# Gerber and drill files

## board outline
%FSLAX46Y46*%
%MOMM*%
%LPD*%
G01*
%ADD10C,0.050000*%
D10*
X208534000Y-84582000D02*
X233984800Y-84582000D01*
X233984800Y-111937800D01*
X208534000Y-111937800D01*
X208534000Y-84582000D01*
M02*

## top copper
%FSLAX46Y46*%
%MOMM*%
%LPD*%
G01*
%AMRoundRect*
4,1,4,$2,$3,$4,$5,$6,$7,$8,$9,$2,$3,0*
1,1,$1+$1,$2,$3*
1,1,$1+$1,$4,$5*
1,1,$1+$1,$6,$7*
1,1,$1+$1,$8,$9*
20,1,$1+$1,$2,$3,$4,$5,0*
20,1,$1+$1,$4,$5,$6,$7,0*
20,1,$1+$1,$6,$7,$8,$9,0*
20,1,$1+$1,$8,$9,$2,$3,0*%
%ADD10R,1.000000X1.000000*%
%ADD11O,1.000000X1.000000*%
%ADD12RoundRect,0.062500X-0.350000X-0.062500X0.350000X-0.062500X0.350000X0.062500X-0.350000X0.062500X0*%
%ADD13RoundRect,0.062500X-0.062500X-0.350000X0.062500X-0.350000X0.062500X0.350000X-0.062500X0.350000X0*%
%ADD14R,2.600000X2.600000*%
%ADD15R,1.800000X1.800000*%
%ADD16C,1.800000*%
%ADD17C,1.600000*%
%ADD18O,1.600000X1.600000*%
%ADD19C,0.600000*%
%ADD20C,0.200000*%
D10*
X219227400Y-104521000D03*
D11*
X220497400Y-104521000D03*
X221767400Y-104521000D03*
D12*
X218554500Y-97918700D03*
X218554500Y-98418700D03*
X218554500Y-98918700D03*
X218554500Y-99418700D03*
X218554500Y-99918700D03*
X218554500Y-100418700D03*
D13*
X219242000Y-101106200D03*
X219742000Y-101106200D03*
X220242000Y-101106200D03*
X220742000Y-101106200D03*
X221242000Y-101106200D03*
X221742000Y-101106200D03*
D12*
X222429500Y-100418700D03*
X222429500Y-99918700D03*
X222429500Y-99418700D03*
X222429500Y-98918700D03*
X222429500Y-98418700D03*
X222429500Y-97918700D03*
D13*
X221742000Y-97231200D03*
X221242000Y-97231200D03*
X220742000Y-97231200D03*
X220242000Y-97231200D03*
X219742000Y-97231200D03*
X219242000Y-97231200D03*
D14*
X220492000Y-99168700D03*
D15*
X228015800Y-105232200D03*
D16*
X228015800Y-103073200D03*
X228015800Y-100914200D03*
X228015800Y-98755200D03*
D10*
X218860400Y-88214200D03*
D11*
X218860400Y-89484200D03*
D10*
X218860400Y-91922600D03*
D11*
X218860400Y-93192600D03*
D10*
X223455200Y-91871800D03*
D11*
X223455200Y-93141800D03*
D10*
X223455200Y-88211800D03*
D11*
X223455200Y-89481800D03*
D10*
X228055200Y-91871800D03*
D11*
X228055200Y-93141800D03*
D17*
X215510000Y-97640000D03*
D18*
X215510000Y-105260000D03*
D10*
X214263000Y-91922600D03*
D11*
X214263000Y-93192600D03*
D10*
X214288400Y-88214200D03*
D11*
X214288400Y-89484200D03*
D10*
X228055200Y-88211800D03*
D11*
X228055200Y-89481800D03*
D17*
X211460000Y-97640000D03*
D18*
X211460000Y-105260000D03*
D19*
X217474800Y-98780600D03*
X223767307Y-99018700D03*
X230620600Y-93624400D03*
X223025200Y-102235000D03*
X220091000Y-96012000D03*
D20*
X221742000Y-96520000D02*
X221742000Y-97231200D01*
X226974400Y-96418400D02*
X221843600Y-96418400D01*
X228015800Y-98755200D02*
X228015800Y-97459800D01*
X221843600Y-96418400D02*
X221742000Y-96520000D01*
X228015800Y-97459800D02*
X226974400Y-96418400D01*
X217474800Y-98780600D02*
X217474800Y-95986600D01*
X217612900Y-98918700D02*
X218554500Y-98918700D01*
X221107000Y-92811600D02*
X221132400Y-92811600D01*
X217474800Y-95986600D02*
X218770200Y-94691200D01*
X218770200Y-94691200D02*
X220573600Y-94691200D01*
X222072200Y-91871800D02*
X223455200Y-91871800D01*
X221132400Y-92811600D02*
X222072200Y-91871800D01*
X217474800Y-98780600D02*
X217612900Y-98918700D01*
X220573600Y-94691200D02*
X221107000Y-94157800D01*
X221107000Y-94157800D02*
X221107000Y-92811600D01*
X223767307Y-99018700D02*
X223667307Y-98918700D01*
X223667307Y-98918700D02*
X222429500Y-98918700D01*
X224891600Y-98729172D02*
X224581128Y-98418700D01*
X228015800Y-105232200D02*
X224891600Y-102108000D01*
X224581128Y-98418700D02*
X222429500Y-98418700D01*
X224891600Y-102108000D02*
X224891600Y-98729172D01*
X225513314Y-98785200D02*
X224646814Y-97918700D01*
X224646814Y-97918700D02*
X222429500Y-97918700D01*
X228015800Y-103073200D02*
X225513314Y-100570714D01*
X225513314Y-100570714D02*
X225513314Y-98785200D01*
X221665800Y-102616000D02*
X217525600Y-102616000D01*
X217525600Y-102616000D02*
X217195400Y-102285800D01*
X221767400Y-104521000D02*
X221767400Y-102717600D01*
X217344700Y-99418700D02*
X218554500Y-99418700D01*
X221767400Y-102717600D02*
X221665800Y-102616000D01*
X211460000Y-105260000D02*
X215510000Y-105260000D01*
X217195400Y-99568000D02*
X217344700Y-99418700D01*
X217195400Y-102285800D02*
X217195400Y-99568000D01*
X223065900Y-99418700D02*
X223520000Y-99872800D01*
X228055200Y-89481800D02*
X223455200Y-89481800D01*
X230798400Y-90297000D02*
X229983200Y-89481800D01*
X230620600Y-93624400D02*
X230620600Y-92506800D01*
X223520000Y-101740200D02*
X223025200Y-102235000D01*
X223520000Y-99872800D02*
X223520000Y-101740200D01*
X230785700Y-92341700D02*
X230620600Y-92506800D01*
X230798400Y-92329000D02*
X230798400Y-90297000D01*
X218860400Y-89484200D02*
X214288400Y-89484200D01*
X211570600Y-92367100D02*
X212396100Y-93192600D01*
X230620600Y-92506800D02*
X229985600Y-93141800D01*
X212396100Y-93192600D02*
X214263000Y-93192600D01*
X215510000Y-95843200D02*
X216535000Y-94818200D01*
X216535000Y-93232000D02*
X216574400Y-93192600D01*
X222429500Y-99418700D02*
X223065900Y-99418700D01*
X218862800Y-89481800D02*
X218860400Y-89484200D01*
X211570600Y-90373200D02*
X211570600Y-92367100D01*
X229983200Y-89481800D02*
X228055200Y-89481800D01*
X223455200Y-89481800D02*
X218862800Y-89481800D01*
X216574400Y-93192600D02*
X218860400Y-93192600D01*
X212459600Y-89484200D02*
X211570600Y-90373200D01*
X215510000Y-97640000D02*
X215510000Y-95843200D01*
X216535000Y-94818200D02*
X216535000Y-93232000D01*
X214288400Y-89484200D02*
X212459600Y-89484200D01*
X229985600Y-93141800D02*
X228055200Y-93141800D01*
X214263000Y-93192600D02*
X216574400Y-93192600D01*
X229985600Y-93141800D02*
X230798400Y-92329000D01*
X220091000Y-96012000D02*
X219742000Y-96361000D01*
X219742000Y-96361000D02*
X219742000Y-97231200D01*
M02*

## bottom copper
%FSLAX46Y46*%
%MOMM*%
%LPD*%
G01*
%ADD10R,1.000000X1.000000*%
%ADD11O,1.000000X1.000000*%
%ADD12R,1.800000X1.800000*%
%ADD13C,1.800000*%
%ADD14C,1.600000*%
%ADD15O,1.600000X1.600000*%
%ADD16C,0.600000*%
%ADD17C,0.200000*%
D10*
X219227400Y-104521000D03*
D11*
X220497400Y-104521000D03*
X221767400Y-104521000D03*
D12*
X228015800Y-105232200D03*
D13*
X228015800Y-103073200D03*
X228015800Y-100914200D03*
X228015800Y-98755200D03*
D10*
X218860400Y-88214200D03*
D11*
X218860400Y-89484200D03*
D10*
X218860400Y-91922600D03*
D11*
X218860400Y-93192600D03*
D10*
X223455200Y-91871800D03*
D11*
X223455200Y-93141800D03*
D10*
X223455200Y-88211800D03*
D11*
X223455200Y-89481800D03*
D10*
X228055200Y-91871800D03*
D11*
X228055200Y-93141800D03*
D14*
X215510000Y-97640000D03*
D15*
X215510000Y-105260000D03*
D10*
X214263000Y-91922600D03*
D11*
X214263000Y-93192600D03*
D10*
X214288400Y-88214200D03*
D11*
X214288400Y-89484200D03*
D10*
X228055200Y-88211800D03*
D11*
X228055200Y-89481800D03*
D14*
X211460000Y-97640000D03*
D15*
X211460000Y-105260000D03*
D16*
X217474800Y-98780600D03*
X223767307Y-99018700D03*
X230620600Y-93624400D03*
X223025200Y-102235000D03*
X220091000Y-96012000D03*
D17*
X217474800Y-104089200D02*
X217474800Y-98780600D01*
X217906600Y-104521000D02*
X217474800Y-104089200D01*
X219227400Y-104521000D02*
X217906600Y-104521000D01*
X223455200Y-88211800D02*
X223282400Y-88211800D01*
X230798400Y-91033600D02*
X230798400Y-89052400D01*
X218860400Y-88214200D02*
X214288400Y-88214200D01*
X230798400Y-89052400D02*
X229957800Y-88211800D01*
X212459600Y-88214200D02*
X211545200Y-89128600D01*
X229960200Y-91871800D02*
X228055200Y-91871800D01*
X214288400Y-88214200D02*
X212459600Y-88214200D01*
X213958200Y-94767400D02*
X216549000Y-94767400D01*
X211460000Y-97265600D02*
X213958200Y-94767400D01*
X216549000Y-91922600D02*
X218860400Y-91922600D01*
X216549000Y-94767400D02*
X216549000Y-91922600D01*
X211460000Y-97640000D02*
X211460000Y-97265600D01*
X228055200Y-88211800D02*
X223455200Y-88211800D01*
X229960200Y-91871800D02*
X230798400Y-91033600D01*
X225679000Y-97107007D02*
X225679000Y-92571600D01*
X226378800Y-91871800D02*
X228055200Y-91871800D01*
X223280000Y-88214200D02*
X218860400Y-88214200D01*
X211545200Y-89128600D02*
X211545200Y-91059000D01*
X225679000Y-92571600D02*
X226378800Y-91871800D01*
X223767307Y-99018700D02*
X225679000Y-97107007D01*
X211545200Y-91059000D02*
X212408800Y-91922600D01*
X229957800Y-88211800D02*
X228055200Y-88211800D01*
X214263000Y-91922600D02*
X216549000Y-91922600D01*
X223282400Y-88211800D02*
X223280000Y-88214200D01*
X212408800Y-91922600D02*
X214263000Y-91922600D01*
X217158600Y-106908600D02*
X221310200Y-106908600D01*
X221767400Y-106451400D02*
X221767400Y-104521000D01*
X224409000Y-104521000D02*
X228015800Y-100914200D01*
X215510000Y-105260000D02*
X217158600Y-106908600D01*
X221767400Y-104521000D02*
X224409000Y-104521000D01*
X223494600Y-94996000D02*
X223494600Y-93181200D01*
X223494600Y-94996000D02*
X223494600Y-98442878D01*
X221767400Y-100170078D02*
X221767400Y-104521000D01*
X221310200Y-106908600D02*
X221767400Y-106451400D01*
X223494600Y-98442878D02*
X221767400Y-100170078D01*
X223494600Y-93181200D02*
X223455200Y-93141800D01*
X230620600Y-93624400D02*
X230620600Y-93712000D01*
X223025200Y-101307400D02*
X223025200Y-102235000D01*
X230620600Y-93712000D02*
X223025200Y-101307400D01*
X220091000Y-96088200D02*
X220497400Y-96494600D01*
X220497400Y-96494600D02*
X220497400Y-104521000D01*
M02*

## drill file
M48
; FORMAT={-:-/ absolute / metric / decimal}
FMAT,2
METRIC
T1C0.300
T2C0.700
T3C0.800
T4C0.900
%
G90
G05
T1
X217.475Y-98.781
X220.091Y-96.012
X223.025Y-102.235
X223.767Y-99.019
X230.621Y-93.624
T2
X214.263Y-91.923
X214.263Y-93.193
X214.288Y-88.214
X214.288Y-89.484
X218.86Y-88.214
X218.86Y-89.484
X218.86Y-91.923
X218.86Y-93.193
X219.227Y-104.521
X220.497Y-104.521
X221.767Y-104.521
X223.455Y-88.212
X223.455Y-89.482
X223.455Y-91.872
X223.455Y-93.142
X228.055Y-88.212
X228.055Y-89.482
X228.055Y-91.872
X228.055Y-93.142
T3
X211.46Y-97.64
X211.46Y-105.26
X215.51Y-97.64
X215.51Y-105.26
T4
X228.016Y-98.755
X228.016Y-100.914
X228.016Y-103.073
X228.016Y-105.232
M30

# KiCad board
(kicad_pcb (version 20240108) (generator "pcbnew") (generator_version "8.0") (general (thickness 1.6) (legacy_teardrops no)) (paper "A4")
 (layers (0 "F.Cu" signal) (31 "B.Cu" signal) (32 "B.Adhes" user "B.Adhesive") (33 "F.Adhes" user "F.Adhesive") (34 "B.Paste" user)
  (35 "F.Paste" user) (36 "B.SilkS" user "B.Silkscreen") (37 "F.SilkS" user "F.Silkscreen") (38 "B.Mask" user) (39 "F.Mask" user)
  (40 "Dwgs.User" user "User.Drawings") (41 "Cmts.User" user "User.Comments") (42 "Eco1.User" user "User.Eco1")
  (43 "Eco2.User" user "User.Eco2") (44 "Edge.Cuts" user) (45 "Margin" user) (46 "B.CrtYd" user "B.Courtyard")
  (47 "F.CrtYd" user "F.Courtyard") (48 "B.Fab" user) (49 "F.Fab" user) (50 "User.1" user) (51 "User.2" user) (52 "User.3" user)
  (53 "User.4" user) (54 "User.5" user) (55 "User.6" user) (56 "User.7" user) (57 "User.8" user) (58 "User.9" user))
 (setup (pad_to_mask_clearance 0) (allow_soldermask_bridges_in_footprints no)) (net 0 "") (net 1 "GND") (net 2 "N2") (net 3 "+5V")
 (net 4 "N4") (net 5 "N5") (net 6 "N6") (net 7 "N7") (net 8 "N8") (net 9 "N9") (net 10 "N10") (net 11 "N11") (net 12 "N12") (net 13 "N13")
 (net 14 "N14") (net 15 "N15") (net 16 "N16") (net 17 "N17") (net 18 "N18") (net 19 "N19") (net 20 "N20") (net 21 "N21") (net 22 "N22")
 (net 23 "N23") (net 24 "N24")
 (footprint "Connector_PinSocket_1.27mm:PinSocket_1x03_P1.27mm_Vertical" (layer "F.Cu") (at 219.2274 104.521 90)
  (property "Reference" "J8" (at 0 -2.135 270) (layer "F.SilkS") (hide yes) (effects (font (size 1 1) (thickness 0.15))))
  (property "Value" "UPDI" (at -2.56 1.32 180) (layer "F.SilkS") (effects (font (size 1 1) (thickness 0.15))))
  (pad "1" thru_hole rect (at 0 0 90) (size 1 1) (drill 0.7) (layers "*.Cu" "*.Mask") (remove_unused_layers no) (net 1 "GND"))
  (pad "2" thru_hole oval (at 0 1.27 90) (size 1 1) (drill 0.7) (layers "*.Cu" "*.Mask") (remove_unused_layers no) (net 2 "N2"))
  (pad "3" thru_hole oval (at 0 2.54 90) (size 1 1) (drill 0.7) (layers "*.Cu" "*.Mask") (remove_unused_layers no) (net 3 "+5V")))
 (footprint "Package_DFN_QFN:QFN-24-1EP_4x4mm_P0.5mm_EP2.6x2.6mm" (layer "F.Cu") (at 220.492 99.1687)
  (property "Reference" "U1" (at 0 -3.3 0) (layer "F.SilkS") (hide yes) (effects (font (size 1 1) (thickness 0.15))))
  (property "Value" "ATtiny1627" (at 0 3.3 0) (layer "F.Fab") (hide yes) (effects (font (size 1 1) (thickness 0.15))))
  (pad "" smd roundrect (at -0.65 -0.65) (size 1.05 1.05) (layers "F.Paste") (roundrect_rratio 0.238095))
  (pad "" smd roundrect (at -0.65 0.65) (size 1.05 1.05) (layers "F.Paste") (roundrect_rratio 0.238095))
  (pad "" smd roundrect (at 0.65 -0.65) (size 1.05 1.05) (layers "F.Paste") (roundrect_rratio 0.238095))
  (pad "" smd roundrect (at 0.65 0.65) (size 1.05 1.05) (layers "F.Paste") (roundrect_rratio 0.238095))
  (pad "1" smd roundrect (at -1.9375 -1.25) (size 0.825 0.25) (layers "F.Cu" "F.Paste" "F.Mask") (roundrect_rratio 0.25) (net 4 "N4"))
  (pad "2" smd roundrect (at -1.9375 -0.75) (size 0.825 0.25) (layers "F.Cu" "F.Paste" "F.Mask") (roundrect_rratio 0.25) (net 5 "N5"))
  (pad "3" smd roundrect (at -1.9375 -0.25) (size 0.825 0.25) (layers "F.Cu" "F.Paste" "F.Mask") (roundrect_rratio 0.25) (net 1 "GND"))
  (pad "4" smd roundrect (at -1.9375 0.25) (size 0.825 0.25) (layers "F.Cu" "F.Paste" "F.Mask") (roundrect_rratio 0.25) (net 3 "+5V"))
  (pad "5" smd roundrect (at -1.9375 0.75) (size 0.825 0.25) (layers "F.Cu" "F.Paste" "F.Mask") (roundrect_rratio 0.25) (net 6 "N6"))
  (pad "6" smd roundrect (at -1.9375 1.25) (size 0.825 0.25) (layers "F.Cu" "F.Paste" "F.Mask") (roundrect_rratio 0.25) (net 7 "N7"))
  (pad "7" smd roundrect (at -1.25 1.9375) (size 0.25 0.825) (layers "F.Cu" "F.Paste" "F.Mask") (roundrect_rratio 0.25) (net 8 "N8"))
  (pad "8" smd roundrect (at -0.75 1.9375) (size 0.25 0.825) (layers "F.Cu" "F.Paste" "F.Mask") (roundrect_rratio 0.25) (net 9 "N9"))
  (pad "9" smd roundrect (at -0.25 1.9375) (size 0.25 0.825) (layers "F.Cu" "F.Paste" "F.Mask") (roundrect_rratio 0.25) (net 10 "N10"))
  (pad "10" smd roundrect (at 0.25 1.9375) (size 0.25 0.825) (layers "F.Cu" "F.Paste" "F.Mask") (roundrect_rratio 0.25) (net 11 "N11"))
  (pad "11" smd roundrect (at 0.75 1.9375) (size 0.25 0.825) (layers "F.Cu" "F.Paste" "F.Mask") (roundrect_rratio 0.25) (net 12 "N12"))
  (pad "12" smd roundrect (at 1.25 1.9375) (size 0.25 0.825) (layers "F.Cu" "F.Paste" "F.Mask") (roundrect_rratio 0.25) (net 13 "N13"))
  (pad "13" smd roundrect (at 1.9375 1.25) (size 0.825 0.25) (layers "F.Cu" "F.Paste" "F.Mask") (roundrect_rratio 0.25) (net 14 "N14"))
  (pad "14" smd roundrect (at 1.9375 0.75) (size 0.825 0.25) (layers "F.Cu" "F.Paste" "F.Mask") (roundrect_rratio 0.25) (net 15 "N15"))
  (pad "15" smd roundrect (at 1.9375 0.25) (size 0.825 0.25) (layers "F.Cu" "F.Paste" "F.Mask") (roundrect_rratio 0.25) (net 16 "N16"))
  (pad "16" smd roundrect (at 1.9375 -0.25) (size 0.825 0.25) (layers "F.Cu" "F.Paste" "F.Mask") (roundrect_rratio 0.25) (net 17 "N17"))
  (pad "17" smd roundrect (at 1.9375 -0.75) (size 0.825 0.25) (layers "F.Cu" "F.Paste" "F.Mask") (roundrect_rratio 0.25) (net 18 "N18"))
  (pad "18" smd roundrect (at 1.9375 -1.25) (size 0.825 0.25) (layers "F.Cu" "F.Paste" "F.Mask") (roundrect_rratio 0.25) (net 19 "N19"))
  (pad "19" smd roundrect (at 1.25 -1.9375) (size 0.25 0.825) (layers "F.Cu" "F.Paste" "F.Mask") (roundrect_rratio 0.25) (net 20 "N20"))
  (pad "20" smd roundrect (at 0.75 -1.9375) (size 0.25 0.825) (layers "F.Cu" "F.Paste" "F.Mask") (roundrect_rratio 0.25) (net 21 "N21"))
  (pad "21" smd roundrect (at 0.25 -1.9375) (size 0.25 0.825) (layers "F.Cu" "F.Paste" "F.Mask") (roundrect_rratio 0.25) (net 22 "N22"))
  (pad "22" smd roundrect (at -0.25 -1.9375) (size 0.25 0.825) (layers "F.Cu" "F.Paste" "F.Mask") (roundrect_rratio 0.25) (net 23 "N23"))
  (pad "23" smd roundrect (at -0.75 -1.9375) (size 0.25 0.825) (layers "F.Cu" "F.Paste" "F.Mask") (roundrect_rratio 0.25) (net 2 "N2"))
  (pad "24" smd roundrect (at -1.25 -1.9375) (size 0.25 0.825) (layers "F.Cu" "F.Paste" "F.Mask") (roundrect_rratio 0.25) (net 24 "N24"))
  (pad "25" smd rect (at 0 0) (size 2.6 2.6) (layers "F.Cu" "F.Mask") (zone_connect 2)))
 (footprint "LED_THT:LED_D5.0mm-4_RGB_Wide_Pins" (layer "F.Cu") (at 228.0158 105.2322 90)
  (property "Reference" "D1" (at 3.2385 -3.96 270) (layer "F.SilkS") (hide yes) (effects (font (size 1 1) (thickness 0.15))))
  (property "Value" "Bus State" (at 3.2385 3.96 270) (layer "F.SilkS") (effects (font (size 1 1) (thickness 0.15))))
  (pad "1" thru_hole rect (at 0 0 90) (size 1.8 1.8) (drill 0.9) (layers "*.Cu" "*.Mask") (remove_unused_layers no) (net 18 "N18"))
  (pad "2" thru_hole circle (at 2.159 0 90) (size 1.8 1.8) (drill 0.9) (layers "*.Cu" "*.Mask") (remove_unused_layers no) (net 19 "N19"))
  (pad "3" thru_hole circle (at 4.318 0 90) (size 1.8 1.8) (drill 0.9) (layers "*.Cu" "*.Mask") (remove_unused_layers no) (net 3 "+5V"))
  (pad "4" thru_hole circle (at 6.477 0 90) (size 1.8 1.8) (drill 0.9) (layers "*.Cu" "*.Mask") (remove_unused_layers no) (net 20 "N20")))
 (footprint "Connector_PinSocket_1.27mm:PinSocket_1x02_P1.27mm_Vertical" (layer "F.Cu") (at 218.8604 88.2142)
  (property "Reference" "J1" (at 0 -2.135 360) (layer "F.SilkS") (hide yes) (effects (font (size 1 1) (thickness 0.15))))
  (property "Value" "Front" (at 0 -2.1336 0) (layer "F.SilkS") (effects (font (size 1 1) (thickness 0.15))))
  (pad "1" thru_hole rect (at 0 0) (size 1 1) (drill 0.7) (layers "*.Cu" "*.Mask") (remove_unused_layers no) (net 17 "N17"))
  (pad "2" thru_hole oval (at 0 1.27) (size 1 1) (drill 0.7) (layers "*.Cu" "*.Mask") (remove_unused_layers no) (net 16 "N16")))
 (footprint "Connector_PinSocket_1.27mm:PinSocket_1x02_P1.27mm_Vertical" (layer "F.Cu") (at 218.8604 91.9226)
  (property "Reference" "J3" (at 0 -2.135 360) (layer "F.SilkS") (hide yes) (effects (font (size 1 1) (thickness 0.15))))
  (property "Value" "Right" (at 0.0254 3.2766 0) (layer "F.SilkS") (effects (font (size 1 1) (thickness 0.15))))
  (pad "1" thru_hole rect (at 0 0) (size 1 1) (drill 0.7) (layers "*.Cu" "*.Mask") (remove_unused_layers no) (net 17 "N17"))
  (pad "2" thru_hole oval (at 0 1.27) (size 1 1) (drill 0.7) (layers "*.Cu" "*.Mask") (remove_unused_layers no) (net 16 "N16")))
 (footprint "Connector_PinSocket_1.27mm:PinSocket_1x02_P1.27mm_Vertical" (layer "F.Cu") (at 223.4552 91.8718)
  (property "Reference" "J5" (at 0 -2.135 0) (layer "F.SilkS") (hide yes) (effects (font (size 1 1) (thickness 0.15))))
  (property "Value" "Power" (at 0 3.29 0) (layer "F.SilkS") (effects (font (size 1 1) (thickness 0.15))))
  (pad "1" thru_hole rect (at 0 0) (size 1 1) (drill 0.7) (layers "*.Cu" "*.Mask") (remove_unused_layers no) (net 1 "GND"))
  (pad "2" thru_hole oval (at 0 1.27) (size 1 1) (drill 0.7) (layers "*.Cu" "*.Mask") (remove_unused_layers no) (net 3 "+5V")))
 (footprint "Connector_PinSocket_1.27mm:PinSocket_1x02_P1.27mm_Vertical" (layer "F.Cu") (at 223.4552 88.2118)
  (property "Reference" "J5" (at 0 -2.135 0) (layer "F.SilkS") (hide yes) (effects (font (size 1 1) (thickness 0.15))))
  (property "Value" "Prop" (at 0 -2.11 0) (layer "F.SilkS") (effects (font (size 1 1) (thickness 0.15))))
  (pad "1" thru_hole rect (at 0 0) (size 1 1) (drill 0.7) (layers "*.Cu" "*.Mask") (remove_unused_layers no) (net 17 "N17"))
  (pad "2" thru_hole oval (at 0 1.27) (size 1 1) (drill 0.7) (layers "*.Cu" "*.Mask") (remove_unused_layers no) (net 16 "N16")))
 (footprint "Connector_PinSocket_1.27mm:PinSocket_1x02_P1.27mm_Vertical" (layer "F.Cu") (at 228.0552 91.8718)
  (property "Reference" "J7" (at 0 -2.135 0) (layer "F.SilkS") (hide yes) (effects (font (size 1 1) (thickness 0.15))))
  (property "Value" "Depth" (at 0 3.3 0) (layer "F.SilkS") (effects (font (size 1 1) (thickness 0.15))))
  (pad "1" thru_hole rect (at 0 0) (size 1 1) (drill 0.7) (layers "*.Cu" "*.Mask") (remove_unused_layers no) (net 17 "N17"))
  (pad "2" thru_hole oval (at 0 1.27) (size 1 1) (drill 0.7) (layers "*.Cu" "*.Mask") (remove_unused_layers no) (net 16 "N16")))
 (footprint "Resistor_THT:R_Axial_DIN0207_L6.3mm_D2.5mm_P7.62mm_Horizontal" (layer "F.Cu") (at 215.51 97.64 -90)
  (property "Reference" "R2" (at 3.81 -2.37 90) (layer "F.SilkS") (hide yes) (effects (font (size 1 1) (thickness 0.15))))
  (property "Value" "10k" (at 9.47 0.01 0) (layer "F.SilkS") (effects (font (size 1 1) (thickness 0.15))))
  (pad "1" thru_hole circle (at 0 0 270) (size 1.6 1.6) (drill 0.8) (layers "*.Cu" "*.Mask") (remove_unused_layers no) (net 16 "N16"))
  (pad "2" thru_hole oval (at 7.62 0 270) (size 1.6 1.6) (drill 0.8) (layers "*.Cu" "*.Mask") (remove_unused_layers no) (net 3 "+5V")))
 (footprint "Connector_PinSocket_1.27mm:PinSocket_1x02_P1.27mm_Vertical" (layer "F.Cu") (at 214.263 91.9226)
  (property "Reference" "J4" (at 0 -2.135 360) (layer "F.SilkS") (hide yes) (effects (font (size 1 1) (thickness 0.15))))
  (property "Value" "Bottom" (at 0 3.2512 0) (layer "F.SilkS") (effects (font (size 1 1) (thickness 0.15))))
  (pad "1" thru_hole rect (at 0 0) (size 1 1) (drill 0.7) (layers "*.Cu" "*.Mask") (remove_unused_layers no) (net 17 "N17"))
  (pad "2" thru_hole oval (at 0 1.27) (size 1 1) (drill 0.7) (layers "*.Cu" "*.Mask") (remove_unused_layers no) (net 16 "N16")))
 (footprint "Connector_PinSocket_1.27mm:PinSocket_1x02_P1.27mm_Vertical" (layer "F.Cu") (at 214.2884 88.2142)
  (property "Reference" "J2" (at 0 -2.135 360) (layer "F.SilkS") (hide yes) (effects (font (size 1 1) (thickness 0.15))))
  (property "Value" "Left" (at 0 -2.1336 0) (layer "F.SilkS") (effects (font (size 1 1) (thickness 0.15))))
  (pad "1" thru_hole rect (at 0 0) (size 1 1) (drill 0.7) (layers "*.Cu" "*.Mask") (remove_unused_layers no) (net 17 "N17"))
  (pad "2" thru_hole oval (at 0 1.27) (size 1 1) (drill 0.7) (layers "*.Cu" "*.Mask") (remove_unused_layers no) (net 16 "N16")))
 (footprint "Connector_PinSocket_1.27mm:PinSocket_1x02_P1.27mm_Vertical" (layer "F.Cu") (at 228.0552 88.2118)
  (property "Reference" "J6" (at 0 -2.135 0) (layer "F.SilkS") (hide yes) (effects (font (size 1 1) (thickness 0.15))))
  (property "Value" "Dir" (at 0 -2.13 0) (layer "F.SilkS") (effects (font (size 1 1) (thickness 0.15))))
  (pad "1" thru_hole rect (at 0 0) (size 1 1) (drill 0.7) (layers "*.Cu" "*.Mask") (remove_unused_layers no) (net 17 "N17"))
  (pad "2" thru_hole oval (at 0 1.27) (size 1 1) (drill 0.7) (layers "*.Cu" "*.Mask") (remove_unused_layers no) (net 16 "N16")))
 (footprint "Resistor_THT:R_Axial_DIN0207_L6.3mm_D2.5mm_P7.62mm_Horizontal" (layer "F.Cu") (at 211.46 97.64 -90)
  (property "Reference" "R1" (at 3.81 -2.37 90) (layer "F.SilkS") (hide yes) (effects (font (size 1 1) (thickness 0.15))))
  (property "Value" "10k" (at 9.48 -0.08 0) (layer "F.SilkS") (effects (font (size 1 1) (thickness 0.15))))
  (pad "1" thru_hole circle (at 0 0 270) (size 1.6 1.6) (drill 0.8) (layers "*.Cu" "*.Mask") (remove_unused_layers no) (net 17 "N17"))
  (pad "2" thru_hole oval (at 7.62 0 270) (size 1.6 1.6) (drill 0.8) (layers "*.Cu" "*.Mask") (remove_unused_layers no) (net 3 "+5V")))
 (gr_rect (start 208.534 84.582) (end 233.9848 111.9378) (stroke (width 0.05) (type default)) (fill none) (layer "Edge.Cuts"))
 (segment (start 221.742 96.52) (end 221.742 97.2312) (width 0.2) (layer "F.Cu") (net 20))
 (segment (start 226.9744 96.4184) (end 221.8436 96.4184) (width 0.2) (layer "F.Cu") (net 20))
 (segment (start 228.0158 98.7552) (end 228.0158 97.4598) (width 0.2) (layer "F.Cu") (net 20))
 (segment (start 221.8436 96.4184) (end 221.742 96.52) (width 0.2) (layer "F.Cu") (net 20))
 (segment (start 228.0158 97.4598) (end 226.9744 96.4184) (width 0.2) (layer "F.Cu") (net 20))
 (segment (start 217.4748 98.7806) (end 217.4748 95.9866) (width 0.2) (layer "F.Cu") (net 1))
 (segment (start 217.6129 98.9187) (end 218.5545 98.9187) (width 0.2) (layer "F.Cu") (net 1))
 (segment (start 221.107 92.8116) (end 221.1324 92.8116) (width 0.2) (layer "F.Cu") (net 1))
 (segment (start 217.4748 95.9866) (end 218.7702 94.6912) (width 0.2) (layer "F.Cu") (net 1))
 (segment (start 218.7702 94.6912) (end 220.5736 94.6912) (width 0.2) (layer "F.Cu") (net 1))
 (segment (start 222.0722 91.8718) (end 223.4552 91.8718) (width 0.2) (layer "F.Cu") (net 1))
 (segment (start 221.1324 92.8116) (end 222.0722 91.8718) (width 0.2) (layer "F.Cu") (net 1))
 (segment (start 217.4748 98.7806) (end 217.6129 98.9187) (width 0.2) (layer "F.Cu") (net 1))
 (segment (start 220.5736 94.6912) (end 221.107 94.1578) (width 0.2) (layer "F.Cu") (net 1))
 (segment (start 221.107 94.1578) (end 221.107 92.8116) (width 0.2) (layer "F.Cu") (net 1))
 (via (at 217.4748 98.7806) (size 0.6) (drill 0.3) (layers "F.Cu" "B.Cu") (free yes) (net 1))
 (segment (start 217.4748 104.0892) (end 217.4748 98.7806) (width 0.2) (layer "B.Cu") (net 1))
 (segment (start 217.9066 104.521) (end 217.4748 104.0892) (width 0.2) (layer "B.Cu") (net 1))
 (segment (start 219.2274 104.521) (end 217.9066 104.521) (width 0.2) (layer "B.Cu") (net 1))
 (segment (start 223.767307 99.0187) (end 223.667307 98.9187) (width 0.2) (layer "F.Cu") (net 17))
 (segment (start 223.667307 98.9187) (end 222.4295 98.9187) (width 0.2) (layer "F.Cu") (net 17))
 (via (at 223.767307 99.0187) (size 0.6) (drill 0.3) (layers "F.Cu" "B.Cu") (free yes) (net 17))
 (segment (start 223.4552 88.2118) (end 223.2824 88.2118) (width 0.2) (layer "B.Cu") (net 17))
 (segment (start 230.7984 91.0336) (end 230.7984 89.0524) (width 0.2) (layer "B.Cu") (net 17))
 (segment (start 218.8604 88.2142) (end 214.2884 88.2142) (width 0.2) (layer "B.Cu") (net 17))
 (segment (start 230.7984 89.0524) (end 229.9578 88.2118) (width 0.2) (layer "B.Cu") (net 17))
 (segment (start 212.4596 88.2142) (end 211.5452 89.1286) (width 0.2) (layer "B.Cu") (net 17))
 (segment (start 229.9602 91.8718) (end 228.0552 91.8718) (width 0.2) (layer "B.Cu") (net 17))
 (segment (start 214.2884 88.2142) (end 212.4596 88.2142) (width 0.2) (layer "B.Cu") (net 17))
 (segment (start 213.9582 94.7674) (end 216.549 94.7674) (width 0.2) (layer "B.Cu") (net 17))
 (segment (start 211.46 97.2656) (end 213.9582 94.7674) (width 0.2) (layer "B.Cu") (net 17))
 (segment (start 216.549 91.9226) (end 218.8604 91.9226) (width 0.2) (layer "B.Cu") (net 17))
 (segment (start 216.549 94.7674) (end 216.549 91.9226) (width 0.2) (layer "B.Cu") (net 17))
 (segment (start 211.46 97.64) (end 211.46 97.2656) (width 0.2) (layer "B.Cu") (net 17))
 (segment (start 228.0552 88.2118) (end 223.4552 88.2118) (width 0.2) (layer "B.Cu") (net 17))
 (segment (start 229.9602 91.8718) (end 230.7984 91.0336) (width 0.2) (layer "B.Cu") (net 17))
 (segment (start 225.679 97.107007) (end 225.679 92.5716) (width 0.2) (layer "B.Cu") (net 17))
 (segment (start 226.3788 91.8718) (end 228.0552 91.8718) (width 0.2) (layer "B.Cu") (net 17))
 (segment (start 223.28 88.2142) (end 218.8604 88.2142) (width 0.2) (layer "B.Cu") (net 17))
 (segment (start 211.5452 89.1286) (end 211.5452 91.059) (width 0.2) (layer "B.Cu") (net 17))
 (segment (start 225.679 92.5716) (end 226.3788 91.8718) (width 0.2) (layer "B.Cu") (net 17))
 (segment (start 223.767307 99.0187) (end 225.679 97.107007) (width 0.2) (layer "B.Cu") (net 17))
 (segment (start 211.5452 91.059) (end 212.4088 91.9226) (width 0.2) (layer "B.Cu") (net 17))
 (segment (start 229.9578 88.2118) (end 228.0552 88.2118) (width 0.2) (layer "B.Cu") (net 17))
 (segment (start 214.263 91.9226) (end 216.549 91.9226) (width 0.2) (layer "B.Cu") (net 17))
 (segment (start 223.2824 88.2118) (end 223.28 88.2142) (width 0.2) (layer "B.Cu") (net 17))
 (segment (start 212.4088 91.9226) (end 214.263 91.9226) (width 0.2) (layer "B.Cu") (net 17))
 (segment (start 224.8916 98.729172) (end 224.581128 98.4187) (width 0.2) (layer "F.Cu") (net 18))
 (segment (start 228.0158 105.2322) (end 224.8916 102.108) (width 0.2) (layer "F.Cu") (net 18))
 (segment (start 224.581128 98.4187) (end 222.4295 98.4187) (width 0.2) (layer "F.Cu") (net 18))
 (segment (start 224.8916 102.108) (end 224.8916 98.729172) (width 0.2) (layer "F.Cu") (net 18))
 (segment (start 225.513314 98.7852) (end 224.646814 97.9187) (width 0.2) (layer "F.Cu") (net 19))
 (segment (start 224.646814 97.9187) (end 222.4295 97.9187) (width 0.2) (layer "F.Cu") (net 19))
 (segment (start 228.0158 103.0732) (end 225.513314 100.570714) (width 0.2) (layer "F.Cu") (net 19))
 (segment (start 225.513314 100.570714) (end 225.513314 98.7852) (width 0.2) (layer "F.Cu") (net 19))
 (segment (start 221.6658 102.616) (end 217.5256 102.616) (width 0.2) (layer "F.Cu") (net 3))
 (segment (start 217.5256 102.616) (end 217.1954 102.2858) (width 0.2) (layer "F.Cu") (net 3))
 (segment (start 221.7674 104.521) (end 221.7674 102.7176) (width 0.2) (layer "F.Cu") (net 3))
 (segment (start 217.3447 99.4187) (end 218.5545 99.4187) (width 0.2) (layer "F.Cu") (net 3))
 (segment (start 221.7674 102.7176) (end 221.6658 102.616) (width 0.2) (layer "F.Cu") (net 3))
 (segment (start 211.46 105.26) (end 215.51 105.26) (width 0.2) (layer "F.Cu") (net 3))
 (segment (start 217.1954 99.568) (end 217.3447 99.4187) (width 0.2) (layer "F.Cu") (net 3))
 (segment (start 217.1954 102.2858) (end 217.1954 99.568) (width 0.2) (layer "F.Cu") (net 3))
 (segment (start 217.1586 106.9086) (end 221.3102 106.9086) (width 0.2) (layer "B.Cu") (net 3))
 (segment (start 221.7674 106.4514) (end 221.7674 104.521) (width 0.2) (layer "B.Cu") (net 3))
 (segment (start 224.409 104.521) (end 228.0158 100.9142) (width 0.2) (layer "B.Cu") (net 3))
 (segment (start 215.51 105.26) (end 217.1586 106.9086) (width 0.2) (layer "B.Cu") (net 3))
 (segment (start 221.7674 104.521) (end 224.409 104.521) (width 0.2) (layer "B.Cu") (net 3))
 (segment (start 223.4946 94.996) (end 223.4946 93.1812) (width 0.2) (layer "B.Cu") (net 3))
 (segment (start 223.4946 94.996) (end 223.4946 98.442878) (width 0.2) (layer "B.Cu") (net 3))
 (segment (start 221.7674 100.170078) (end 221.7674 104.521) (width 0.2) (layer "B.Cu") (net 3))
 (segment (start 221.3102 106.9086) (end 221.7674 106.4514) (width 0.2) (layer "B.Cu") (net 3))
 (segment (start 223.4946 98.442878) (end 221.7674 100.170078) (width 0.2) (layer "B.Cu") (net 3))
 (segment (start 223.4946 93.1812) (end 223.4552 93.1418) (width 0.2) (layer "B.Cu") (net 3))
 (segment (start 223.0659 99.4187) (end 223.52 99.8728) (width 0.2) (layer "F.Cu") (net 16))
 (segment (start 228.0552 89.4818) (end 223.4552 89.4818) (width 0.2) (layer "F.Cu") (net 16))
 (segment (start 230.7984 90.297) (end 229.9832 89.4818) (width 0.2) (layer "F.Cu") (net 16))
 (segment (start 230.6206 93.6244) (end 230.6206 92.5068) (width 0.2) (layer "F.Cu") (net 16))
 (segment (start 223.52 101.7402) (end 223.0252 102.235) (width 0.2) (layer "F.Cu") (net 16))
 (segment (start 223.52 99.8728) (end 223.52 101.7402) (width 0.2) (layer "F.Cu") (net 16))
 (segment (start 230.7857 92.3417) (end 230.6206 92.5068) (width 0.2) (layer "F.Cu") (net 16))
 (segment (start 230.7984 92.329) (end 230.7984 90.297) (width 0.2) (layer "F.Cu") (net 16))
 (segment (start 218.8604 89.4842) (end 214.2884 89.4842) (width 0.2) (layer "F.Cu") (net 16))
 (segment (start 211.5706 92.3671) (end 212.3961 93.1926) (width 0.2) (layer "F.Cu") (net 16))
 (segment (start 230.6206 92.5068) (end 229.9856 93.1418) (width 0.2) (layer "F.Cu") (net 16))
 (segment (start 212.3961 93.1926) (end 214.263 93.1926) (width 0.2) (layer "F.Cu") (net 16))
 (segment (start 215.51 95.8432) (end 216.535 94.8182) (width 0.2) (layer "F.Cu") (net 16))
 (segment (start 216.535 93.232) (end 216.5744 93.1926) (width 0.2) (layer "F.Cu") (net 16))
 (segment (start 222.4295 99.4187) (end 223.0659 99.4187) (width 0.2) (layer "F.Cu") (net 16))
 (segment (start 218.8628 89.4818) (end 218.8604 89.4842) (width 0.2) (layer "F.Cu") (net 16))
 (segment (start 211.5706 90.3732) (end 211.5706 92.3671) (width 0.2) (layer "F.Cu") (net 16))
 (segment (start 229.9832 89.4818) (end 228.0552 89.4818) (width 0.2) (layer "F.Cu") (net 16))
 (segment (start 223.4552 89.4818) (end 218.8628 89.4818) (width 0.2) (layer "F.Cu") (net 16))
 (segment (start 216.5744 93.1926) (end 218.8604 93.1926) (width 0.2) (layer "F.Cu") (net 16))
 (segment (start 212.4596 89.4842) (end 211.5706 90.3732) (width 0.2) (layer "F.Cu") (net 16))
 (segment (start 215.51 97.64) (end 215.51 95.8432) (width 0.2) (layer "F.Cu") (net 16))
 (segment (start 216.535 94.8182) (end 216.535 93.232) (width 0.2) (layer "F.Cu") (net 16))
 (segment (start 214.2884 89.4842) (end 212.4596 89.4842) (width 0.2) (layer "F.Cu") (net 16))
 (segment (start 229.9856 93.1418) (end 228.0552 93.1418) (width 0.2) (layer "F.Cu") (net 16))
 (segment (start 214.263 93.1926) (end 216.5744 93.1926) (width 0.2) (layer "F.Cu") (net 16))
 (segment (start 229.9856 93.1418) (end 230.7984 92.329) (width 0.2) (layer "F.Cu") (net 16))
 (via (at 230.6206 93.6244) (size 0.6) (drill 0.3) (layers "F.Cu" "B.Cu") (free yes) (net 16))
 (via (at 223.0252 102.235) (size 0.6) (drill 0.3) (layers "F.Cu" "B.Cu") (free yes) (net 16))
 (segment (start 230.6206 93.6244) (end 230.6206 93.712) (width 0.2) (layer "B.Cu") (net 16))
 (segment (start 223.0252 101.3074) (end 223.0252 102.235) (width 0.2) (layer "B.Cu") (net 16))
 (segment (start 230.6206 93.712) (end 223.0252 101.3074) (width 0.2) (layer "B.Cu") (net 16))
 (segment (start 220.091 96.012) (end 219.742 96.361) (width 0.2) (layer "F.Cu") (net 2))
 (segment (start 219.742 96.361) (end 219.742 97.2312) (width 0.2) (layer "F.Cu") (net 2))
 (via (at 220.091 96.012) (size 0.6) (drill 0.3) (layers "F.Cu" "B.Cu") (free yes) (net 2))
 (segment (start 220.091 96.0882) (end 220.4974 96.4946) (width 0.2) (layer "B.Cu") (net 2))
 (segment (start 220.4974 96.4946) (end 220.4974 104.521) (width 0.2) (layer "B.Cu") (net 2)))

